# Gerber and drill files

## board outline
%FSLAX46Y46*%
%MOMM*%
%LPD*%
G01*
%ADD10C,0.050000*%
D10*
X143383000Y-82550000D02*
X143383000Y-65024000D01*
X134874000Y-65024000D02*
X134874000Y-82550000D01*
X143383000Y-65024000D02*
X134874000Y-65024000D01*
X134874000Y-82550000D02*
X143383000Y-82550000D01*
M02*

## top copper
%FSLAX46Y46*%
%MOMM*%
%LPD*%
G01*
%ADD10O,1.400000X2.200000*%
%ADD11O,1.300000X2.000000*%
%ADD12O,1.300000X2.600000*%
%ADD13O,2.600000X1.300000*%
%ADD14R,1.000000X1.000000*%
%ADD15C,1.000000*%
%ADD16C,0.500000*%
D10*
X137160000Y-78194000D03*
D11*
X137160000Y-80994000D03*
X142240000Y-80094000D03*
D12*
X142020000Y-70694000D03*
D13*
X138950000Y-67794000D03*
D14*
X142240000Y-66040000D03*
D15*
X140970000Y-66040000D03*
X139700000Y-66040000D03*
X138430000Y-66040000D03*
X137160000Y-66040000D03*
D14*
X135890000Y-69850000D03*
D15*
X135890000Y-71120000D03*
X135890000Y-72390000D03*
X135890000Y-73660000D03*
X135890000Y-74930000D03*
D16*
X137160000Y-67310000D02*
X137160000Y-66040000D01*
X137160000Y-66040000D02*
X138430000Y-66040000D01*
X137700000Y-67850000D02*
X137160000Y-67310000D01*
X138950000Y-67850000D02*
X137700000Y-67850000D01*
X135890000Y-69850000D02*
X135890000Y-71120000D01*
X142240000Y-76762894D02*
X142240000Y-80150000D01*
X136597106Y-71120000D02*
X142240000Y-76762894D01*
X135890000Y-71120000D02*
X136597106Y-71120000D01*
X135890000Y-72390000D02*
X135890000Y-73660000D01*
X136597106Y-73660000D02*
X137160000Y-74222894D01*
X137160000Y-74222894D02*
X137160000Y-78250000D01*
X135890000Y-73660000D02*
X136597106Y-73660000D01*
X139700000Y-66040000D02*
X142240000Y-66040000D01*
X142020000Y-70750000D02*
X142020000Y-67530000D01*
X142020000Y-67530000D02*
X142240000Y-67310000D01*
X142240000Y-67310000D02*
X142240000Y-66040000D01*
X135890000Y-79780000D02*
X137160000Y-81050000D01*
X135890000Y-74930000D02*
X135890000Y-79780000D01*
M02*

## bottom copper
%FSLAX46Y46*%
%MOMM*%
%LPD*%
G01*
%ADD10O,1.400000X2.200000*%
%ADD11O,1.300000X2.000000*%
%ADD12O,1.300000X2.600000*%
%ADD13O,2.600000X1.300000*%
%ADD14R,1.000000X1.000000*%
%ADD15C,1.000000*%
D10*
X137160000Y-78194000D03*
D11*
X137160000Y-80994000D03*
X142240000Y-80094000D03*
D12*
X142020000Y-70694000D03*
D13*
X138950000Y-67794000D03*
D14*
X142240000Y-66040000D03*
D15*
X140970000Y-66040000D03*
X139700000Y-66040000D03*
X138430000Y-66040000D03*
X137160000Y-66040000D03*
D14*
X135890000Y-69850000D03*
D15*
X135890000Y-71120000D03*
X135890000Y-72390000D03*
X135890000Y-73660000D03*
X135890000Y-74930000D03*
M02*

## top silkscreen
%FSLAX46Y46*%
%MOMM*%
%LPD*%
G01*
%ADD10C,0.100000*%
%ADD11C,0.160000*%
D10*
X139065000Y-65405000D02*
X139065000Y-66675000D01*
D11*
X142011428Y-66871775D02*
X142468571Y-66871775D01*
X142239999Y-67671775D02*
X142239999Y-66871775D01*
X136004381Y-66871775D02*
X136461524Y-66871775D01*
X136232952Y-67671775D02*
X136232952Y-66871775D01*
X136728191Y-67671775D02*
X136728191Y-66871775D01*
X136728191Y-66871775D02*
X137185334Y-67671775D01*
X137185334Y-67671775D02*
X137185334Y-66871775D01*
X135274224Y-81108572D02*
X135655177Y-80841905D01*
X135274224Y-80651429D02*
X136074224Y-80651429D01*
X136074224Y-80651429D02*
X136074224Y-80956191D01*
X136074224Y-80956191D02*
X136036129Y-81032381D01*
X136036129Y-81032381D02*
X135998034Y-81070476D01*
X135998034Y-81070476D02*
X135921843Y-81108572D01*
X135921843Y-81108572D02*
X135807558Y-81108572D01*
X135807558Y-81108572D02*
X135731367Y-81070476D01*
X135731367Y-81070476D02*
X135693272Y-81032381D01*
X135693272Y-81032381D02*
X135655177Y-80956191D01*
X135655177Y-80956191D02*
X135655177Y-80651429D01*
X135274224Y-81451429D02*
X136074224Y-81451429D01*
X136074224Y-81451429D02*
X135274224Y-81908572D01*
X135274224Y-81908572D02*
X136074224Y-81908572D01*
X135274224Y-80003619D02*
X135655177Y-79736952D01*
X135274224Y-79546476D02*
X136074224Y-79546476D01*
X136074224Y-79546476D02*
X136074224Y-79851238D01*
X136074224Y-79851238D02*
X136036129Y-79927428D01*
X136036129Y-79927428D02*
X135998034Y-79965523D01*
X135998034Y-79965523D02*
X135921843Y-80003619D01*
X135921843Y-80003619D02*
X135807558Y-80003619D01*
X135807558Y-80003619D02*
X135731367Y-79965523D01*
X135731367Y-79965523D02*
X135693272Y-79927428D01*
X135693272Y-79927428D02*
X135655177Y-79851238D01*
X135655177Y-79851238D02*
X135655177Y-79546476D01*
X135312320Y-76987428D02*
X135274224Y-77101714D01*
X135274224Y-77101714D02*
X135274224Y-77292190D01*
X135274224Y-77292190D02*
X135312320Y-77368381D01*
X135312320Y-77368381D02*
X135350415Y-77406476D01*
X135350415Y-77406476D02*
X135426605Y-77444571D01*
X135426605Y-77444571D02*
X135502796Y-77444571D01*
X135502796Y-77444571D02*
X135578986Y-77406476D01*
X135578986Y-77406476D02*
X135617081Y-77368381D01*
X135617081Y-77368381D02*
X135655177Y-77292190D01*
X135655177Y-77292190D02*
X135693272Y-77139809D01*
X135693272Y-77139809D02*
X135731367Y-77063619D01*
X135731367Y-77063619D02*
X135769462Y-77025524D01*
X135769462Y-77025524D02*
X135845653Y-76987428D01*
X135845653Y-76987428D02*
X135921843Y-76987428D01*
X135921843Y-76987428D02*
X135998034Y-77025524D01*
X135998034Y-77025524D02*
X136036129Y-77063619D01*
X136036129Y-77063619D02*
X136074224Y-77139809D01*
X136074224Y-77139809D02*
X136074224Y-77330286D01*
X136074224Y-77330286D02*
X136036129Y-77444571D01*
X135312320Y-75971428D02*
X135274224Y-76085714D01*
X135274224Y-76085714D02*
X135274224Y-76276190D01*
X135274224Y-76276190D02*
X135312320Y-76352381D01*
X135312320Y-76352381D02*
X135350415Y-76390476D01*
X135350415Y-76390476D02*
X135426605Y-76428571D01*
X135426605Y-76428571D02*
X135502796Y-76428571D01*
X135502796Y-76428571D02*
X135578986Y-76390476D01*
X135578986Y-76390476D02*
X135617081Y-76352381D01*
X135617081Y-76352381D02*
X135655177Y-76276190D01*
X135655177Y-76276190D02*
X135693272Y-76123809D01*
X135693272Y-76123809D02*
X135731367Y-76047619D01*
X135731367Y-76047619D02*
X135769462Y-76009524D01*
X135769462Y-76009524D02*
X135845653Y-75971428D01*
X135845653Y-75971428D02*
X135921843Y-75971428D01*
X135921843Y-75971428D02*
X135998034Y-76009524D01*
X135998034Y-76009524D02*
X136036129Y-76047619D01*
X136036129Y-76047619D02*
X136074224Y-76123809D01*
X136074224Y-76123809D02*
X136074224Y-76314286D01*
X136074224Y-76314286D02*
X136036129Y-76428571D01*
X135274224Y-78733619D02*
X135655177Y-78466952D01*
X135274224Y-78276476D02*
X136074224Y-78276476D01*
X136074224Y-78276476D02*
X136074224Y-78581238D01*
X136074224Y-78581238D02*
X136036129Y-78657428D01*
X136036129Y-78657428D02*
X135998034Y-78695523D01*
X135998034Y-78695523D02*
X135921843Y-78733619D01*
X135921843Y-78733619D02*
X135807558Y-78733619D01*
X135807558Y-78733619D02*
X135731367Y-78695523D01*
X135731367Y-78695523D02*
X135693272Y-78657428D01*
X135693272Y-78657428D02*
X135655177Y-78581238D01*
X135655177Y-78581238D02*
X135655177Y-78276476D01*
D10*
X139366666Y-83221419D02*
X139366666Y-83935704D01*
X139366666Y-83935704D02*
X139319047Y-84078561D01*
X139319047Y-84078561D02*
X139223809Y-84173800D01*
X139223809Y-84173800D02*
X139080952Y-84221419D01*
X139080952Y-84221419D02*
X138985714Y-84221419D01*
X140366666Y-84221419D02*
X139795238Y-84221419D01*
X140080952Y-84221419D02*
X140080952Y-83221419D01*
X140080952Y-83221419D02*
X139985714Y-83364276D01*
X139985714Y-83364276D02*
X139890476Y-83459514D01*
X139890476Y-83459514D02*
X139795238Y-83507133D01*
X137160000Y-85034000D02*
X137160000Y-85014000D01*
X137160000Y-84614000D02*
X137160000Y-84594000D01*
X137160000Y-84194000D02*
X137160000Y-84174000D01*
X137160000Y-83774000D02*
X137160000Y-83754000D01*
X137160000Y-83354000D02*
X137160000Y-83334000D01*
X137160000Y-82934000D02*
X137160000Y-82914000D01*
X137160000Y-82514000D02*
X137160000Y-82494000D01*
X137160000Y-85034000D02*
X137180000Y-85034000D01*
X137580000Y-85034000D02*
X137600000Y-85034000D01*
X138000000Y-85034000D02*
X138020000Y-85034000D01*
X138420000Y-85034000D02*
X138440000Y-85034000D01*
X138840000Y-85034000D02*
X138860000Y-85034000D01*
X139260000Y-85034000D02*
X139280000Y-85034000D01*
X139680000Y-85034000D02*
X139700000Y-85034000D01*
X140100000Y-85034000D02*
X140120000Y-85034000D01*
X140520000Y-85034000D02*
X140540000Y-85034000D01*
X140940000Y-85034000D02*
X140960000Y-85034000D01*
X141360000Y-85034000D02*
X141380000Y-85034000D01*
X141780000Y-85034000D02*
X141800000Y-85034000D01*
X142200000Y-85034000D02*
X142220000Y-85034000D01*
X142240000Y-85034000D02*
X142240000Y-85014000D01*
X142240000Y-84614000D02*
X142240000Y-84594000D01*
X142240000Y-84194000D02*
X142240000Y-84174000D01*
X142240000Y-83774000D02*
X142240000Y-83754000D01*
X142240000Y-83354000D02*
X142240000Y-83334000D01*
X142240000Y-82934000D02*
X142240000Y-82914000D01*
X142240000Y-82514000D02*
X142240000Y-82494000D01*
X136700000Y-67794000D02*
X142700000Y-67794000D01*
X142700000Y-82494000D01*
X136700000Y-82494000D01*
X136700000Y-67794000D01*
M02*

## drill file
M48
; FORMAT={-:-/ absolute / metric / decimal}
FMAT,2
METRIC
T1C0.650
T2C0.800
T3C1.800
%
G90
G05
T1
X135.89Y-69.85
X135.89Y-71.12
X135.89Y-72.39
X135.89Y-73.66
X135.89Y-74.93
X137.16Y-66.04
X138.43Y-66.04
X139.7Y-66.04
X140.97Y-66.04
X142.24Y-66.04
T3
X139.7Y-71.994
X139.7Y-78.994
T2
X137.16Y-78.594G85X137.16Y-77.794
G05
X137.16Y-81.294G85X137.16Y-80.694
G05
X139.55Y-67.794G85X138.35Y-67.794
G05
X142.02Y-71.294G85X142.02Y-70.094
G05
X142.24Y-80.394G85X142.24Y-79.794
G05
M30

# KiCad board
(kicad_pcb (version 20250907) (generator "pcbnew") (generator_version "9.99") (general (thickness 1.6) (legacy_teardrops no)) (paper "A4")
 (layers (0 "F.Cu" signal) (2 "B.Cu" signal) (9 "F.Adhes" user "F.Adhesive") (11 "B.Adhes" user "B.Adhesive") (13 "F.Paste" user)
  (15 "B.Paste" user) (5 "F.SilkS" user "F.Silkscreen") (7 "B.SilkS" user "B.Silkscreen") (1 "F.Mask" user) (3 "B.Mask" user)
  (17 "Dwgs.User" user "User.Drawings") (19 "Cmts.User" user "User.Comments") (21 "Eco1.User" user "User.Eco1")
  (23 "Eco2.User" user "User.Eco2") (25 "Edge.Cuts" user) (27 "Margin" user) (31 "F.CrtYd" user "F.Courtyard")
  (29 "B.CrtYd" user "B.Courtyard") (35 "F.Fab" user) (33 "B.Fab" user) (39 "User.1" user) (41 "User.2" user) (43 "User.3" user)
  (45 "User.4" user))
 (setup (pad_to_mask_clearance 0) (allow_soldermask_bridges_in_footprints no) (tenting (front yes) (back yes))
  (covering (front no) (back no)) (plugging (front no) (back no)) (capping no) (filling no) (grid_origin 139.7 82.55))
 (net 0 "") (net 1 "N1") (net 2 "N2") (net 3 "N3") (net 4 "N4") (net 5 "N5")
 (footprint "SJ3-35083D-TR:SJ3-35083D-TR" (layer "F.Cu") (at 139.7 82.494)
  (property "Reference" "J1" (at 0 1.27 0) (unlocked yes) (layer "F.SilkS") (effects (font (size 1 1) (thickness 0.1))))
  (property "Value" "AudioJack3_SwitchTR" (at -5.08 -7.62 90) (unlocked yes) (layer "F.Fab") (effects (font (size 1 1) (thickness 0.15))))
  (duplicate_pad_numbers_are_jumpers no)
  (fp_line (start -2.54 2.54) (end -2.54 0) (stroke (width 0.1) (type dot)) (layer "F.SilkS"))
  (fp_line (start -2.54 2.54) (end 2.54 2.54) (stroke (width 0.1) (type dot)) (layer "F.SilkS"))
  (fp_line (start 2.54 2.54) (end 2.54 0) (stroke (width 0.1) (type dot)) (layer "F.SilkS"))
  (fp_rect (start -3 -14.7) (end 3 0) (stroke (width 0.1) (type solid)) (fill no) (layer "F.SilkS"))
  (pad "" np_thru_hole circle (at 0 -10.5 90) (size 1.8 1.8) (drill 1.8) (layers "*.Cu" "*.Mask") (tenting (front none) (back none)))
  (pad "" np_thru_hole circle (at 0 -3.5 90) (size 1.8 1.8) (drill 1.8) (layers "*.Cu" "*.Mask") (tenting (front none) (back none)))
  (pad "R" thru_hole oval (at -2.54 -4.3 90) (size 2.2 1.4) (drill oval 1.6 0.8) (layers "*.Cu" "*.Mask") (remove_unused_layers no)
   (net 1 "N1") (thermal_bridge_angle 45) (tenting (front none) (back none)))
  (pad "RN" thru_hole oval (at -2.54 -1.5 90) (size 2 1.3) (drill oval 1.4 0.8) (layers "*.Cu" "*.Mask") (remove_unused_layers no)
   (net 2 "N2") (thermal_bridge_angle 45) (tenting (front none) (back none)))
  (pad "S" thru_hole oval (at 2.54 -2.4 90) (size 2 1.3) (drill oval 1.4 0.8) (layers "*.Cu" "*.Mask") (remove_unused_layers no)
   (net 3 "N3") (thermal_bridge_angle 45) (tenting (front none) (back none)))
  (pad "T" thru_hole oval (at 2.32 -11.8 90) (size 2.6 1.3) (drill oval 2 0.8) (layers "*.Cu" "*.Mask") (remove_unused_layers no)
   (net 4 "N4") (thermal_bridge_angle 45) (tenting (front none) (back none)))
  (pad "TN" thru_hole oval (at -0.75 -14.7 180) (size 2.6 1.3) (drill oval 2 0.8) (layers "*.Cu" "*.Mask") (remove_unused_layers no)
   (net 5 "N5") (thermal_bridge_angle 45) (tenting (front none) (back none))))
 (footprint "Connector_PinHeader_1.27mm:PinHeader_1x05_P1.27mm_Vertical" (layer "B.Cu") (at 142.24 66.04 90)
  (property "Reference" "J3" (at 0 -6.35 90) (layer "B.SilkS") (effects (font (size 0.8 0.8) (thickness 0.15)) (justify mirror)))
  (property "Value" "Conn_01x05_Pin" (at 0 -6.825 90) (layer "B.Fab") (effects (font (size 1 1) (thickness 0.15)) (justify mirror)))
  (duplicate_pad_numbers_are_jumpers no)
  (pad "1" thru_hole rect (at 0 0 90) (size 1 1) (drill 0.65) (layers "*.Cu" "*.Mask") (remove_unused_layers no) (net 4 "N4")
   (tenting (front none) (back none)))
  (pad "2" thru_hole circle (at 0 -1.27 90) (size 1 1) (drill 0.65) (layers "*.Cu" "*.Mask") (remove_unused_layers no) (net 4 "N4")
   (tenting (front none) (back none)))
  (pad "3" thru_hole circle (at 0 -2.54 90) (size 1 1) (drill 0.65) (layers "*.Cu" "*.Mask") (remove_unused_layers no) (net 4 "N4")
   (tenting (front none) (back none)))
  (pad "4" thru_hole circle (at 0 -3.81 90) (size 1 1) (drill 0.65) (layers "*.Cu" "*.Mask") (remove_unused_layers no) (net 5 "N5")
   (tenting (front none) (back none)))
  (pad "5" thru_hole circle (at 0 -5.08 90) (size 1 1) (drill 0.65) (layers "*.Cu" "*.Mask") (remove_unused_layers no) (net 5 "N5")
   (tenting (front none) (back none))))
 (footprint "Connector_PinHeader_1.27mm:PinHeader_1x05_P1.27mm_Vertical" (layer "B.Cu") (at 135.89 69.85 180)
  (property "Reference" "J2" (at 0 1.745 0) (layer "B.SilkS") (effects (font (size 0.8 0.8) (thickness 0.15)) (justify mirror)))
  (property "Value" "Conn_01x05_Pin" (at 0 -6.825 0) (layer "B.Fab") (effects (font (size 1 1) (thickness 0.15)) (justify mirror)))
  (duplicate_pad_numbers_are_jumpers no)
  (pad "1" thru_hole rect (at 0 0 180) (size 1 1) (drill 0.65) (layers "*.Cu" "*.Mask") (remove_unused_layers no) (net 3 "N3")
   (tenting (front none) (back none)))
  (pad "2" thru_hole circle (at 0 -1.27 180) (size 1 1) (drill 0.65) (layers "*.Cu" "*.Mask") (remove_unused_layers no) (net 3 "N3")
   (tenting (front none) (back none)))
  (pad "3" thru_hole circle (at 0 -2.54 180) (size 1 1) (drill 0.65) (layers "*.Cu" "*.Mask") (remove_unused_layers no) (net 1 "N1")
   (tenting (front none) (back none)))
  (pad "4" thru_hole circle (at 0 -3.81 180) (size 1 1) (drill 0.65) (layers "*.Cu" "*.Mask") (remove_unused_layers no) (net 1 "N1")
   (tenting (front none) (back none)))
  (pad "5" thru_hole circle (at 0 -5.08 180) (size 1 1) (drill 0.65) (layers "*.Cu" "*.Mask") (remove_unused_layers no) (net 2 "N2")
   (tenting (front none) (back none))))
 (gr_line (start 139.065 65.405) (end 139.065 66.675) (stroke (width 0.1) (type default)) (layer "F.SilkS"))
 (gr_line (start 143.383 82.55) (end 143.383 65.024) (stroke (width 0.05) (type default)) (layer "Edge.Cuts"))
 (gr_line (start 134.874 65.024) (end 134.874 82.55) (stroke (width 0.05) (type default)) (layer "Edge.Cuts"))
 (gr_line (start 143.383 65.024) (end 134.874 65.024) (stroke (width 0.05) (type default)) (layer "Edge.Cuts"))
 (gr_line (start 134.874 82.55) (end 143.383 82.55) (stroke (width 0.05) (type default)) (layer "Edge.Cuts"))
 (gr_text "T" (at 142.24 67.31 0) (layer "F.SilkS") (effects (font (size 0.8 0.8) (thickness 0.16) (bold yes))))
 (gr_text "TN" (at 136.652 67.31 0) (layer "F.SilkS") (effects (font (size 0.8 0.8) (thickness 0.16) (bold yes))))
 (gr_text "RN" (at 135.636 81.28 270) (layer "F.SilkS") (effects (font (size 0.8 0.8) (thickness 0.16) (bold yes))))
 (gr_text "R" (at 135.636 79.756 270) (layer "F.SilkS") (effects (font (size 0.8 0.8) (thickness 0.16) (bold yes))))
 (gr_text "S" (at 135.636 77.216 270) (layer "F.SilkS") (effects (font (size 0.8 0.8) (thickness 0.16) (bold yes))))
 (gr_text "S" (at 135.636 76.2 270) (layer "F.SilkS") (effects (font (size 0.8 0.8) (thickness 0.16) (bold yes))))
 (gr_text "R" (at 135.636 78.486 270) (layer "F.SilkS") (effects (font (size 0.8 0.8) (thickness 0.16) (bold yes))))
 (segment (start 137.16 67.31) (end 137.16 66.04) (width 0.5) (layer "F.Cu") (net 5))
 (segment (start 137.16 66.04) (end 138.43 66.04) (width 0.5) (layer "F.Cu") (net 5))
 (segment (start 137.7 67.85) (end 137.16 67.31) (width 0.5) (layer "F.Cu") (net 5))
 (segment (start 138.95 67.85) (end 137.7 67.85) (width 0.5) (layer "F.Cu") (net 5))
 (segment (start 135.89 69.85) (end 135.89 71.12) (width 0.5) (layer "F.Cu") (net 3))
 (segment (start 142.24 76.762894) (end 142.24 80.15) (width 0.5) (layer "F.Cu") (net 3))
 (segment (start 136.597106 71.12) (end 142.24 76.762894) (width 0.5) (layer "F.Cu") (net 3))
 (segment (start 135.89 71.12) (end 136.597106 71.12) (width 0.5) (layer "F.Cu") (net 3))
 (segment (start 135.89 72.39) (end 135.89 73.66) (width 0.5) (layer "F.Cu") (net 1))
 (segment (start 136.597106 73.66) (end 137.16 74.222894) (width 0.5) (layer "F.Cu") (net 1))
 (segment (start 137.16 74.222894) (end 137.16 78.25) (width 0.5) (layer "F.Cu") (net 1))
 (segment (start 135.89 73.66) (end 136.597106 73.66) (width 0.5) (layer "F.Cu") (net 1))
 (segment (start 139.7 66.04) (end 142.24 66.04) (width 0.5) (layer "F.Cu") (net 4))
 (segment (start 142.02 70.75) (end 142.02 67.53) (width 0.5) (layer "F.Cu") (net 4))
 (segment (start 142.02 67.53) (end 142.24 67.31) (width 0.5) (layer "F.Cu") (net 4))
 (segment (start 142.24 67.31) (end 142.24 66.04) (width 0.5) (layer "F.Cu") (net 4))
 (segment (start 135.89 79.78) (end 137.16 81.05) (width 0.5) (layer "F.Cu") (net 2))
 (segment (start 135.89 74.93) (end 135.89 79.78) (width 0.5) (layer "F.Cu") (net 2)))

